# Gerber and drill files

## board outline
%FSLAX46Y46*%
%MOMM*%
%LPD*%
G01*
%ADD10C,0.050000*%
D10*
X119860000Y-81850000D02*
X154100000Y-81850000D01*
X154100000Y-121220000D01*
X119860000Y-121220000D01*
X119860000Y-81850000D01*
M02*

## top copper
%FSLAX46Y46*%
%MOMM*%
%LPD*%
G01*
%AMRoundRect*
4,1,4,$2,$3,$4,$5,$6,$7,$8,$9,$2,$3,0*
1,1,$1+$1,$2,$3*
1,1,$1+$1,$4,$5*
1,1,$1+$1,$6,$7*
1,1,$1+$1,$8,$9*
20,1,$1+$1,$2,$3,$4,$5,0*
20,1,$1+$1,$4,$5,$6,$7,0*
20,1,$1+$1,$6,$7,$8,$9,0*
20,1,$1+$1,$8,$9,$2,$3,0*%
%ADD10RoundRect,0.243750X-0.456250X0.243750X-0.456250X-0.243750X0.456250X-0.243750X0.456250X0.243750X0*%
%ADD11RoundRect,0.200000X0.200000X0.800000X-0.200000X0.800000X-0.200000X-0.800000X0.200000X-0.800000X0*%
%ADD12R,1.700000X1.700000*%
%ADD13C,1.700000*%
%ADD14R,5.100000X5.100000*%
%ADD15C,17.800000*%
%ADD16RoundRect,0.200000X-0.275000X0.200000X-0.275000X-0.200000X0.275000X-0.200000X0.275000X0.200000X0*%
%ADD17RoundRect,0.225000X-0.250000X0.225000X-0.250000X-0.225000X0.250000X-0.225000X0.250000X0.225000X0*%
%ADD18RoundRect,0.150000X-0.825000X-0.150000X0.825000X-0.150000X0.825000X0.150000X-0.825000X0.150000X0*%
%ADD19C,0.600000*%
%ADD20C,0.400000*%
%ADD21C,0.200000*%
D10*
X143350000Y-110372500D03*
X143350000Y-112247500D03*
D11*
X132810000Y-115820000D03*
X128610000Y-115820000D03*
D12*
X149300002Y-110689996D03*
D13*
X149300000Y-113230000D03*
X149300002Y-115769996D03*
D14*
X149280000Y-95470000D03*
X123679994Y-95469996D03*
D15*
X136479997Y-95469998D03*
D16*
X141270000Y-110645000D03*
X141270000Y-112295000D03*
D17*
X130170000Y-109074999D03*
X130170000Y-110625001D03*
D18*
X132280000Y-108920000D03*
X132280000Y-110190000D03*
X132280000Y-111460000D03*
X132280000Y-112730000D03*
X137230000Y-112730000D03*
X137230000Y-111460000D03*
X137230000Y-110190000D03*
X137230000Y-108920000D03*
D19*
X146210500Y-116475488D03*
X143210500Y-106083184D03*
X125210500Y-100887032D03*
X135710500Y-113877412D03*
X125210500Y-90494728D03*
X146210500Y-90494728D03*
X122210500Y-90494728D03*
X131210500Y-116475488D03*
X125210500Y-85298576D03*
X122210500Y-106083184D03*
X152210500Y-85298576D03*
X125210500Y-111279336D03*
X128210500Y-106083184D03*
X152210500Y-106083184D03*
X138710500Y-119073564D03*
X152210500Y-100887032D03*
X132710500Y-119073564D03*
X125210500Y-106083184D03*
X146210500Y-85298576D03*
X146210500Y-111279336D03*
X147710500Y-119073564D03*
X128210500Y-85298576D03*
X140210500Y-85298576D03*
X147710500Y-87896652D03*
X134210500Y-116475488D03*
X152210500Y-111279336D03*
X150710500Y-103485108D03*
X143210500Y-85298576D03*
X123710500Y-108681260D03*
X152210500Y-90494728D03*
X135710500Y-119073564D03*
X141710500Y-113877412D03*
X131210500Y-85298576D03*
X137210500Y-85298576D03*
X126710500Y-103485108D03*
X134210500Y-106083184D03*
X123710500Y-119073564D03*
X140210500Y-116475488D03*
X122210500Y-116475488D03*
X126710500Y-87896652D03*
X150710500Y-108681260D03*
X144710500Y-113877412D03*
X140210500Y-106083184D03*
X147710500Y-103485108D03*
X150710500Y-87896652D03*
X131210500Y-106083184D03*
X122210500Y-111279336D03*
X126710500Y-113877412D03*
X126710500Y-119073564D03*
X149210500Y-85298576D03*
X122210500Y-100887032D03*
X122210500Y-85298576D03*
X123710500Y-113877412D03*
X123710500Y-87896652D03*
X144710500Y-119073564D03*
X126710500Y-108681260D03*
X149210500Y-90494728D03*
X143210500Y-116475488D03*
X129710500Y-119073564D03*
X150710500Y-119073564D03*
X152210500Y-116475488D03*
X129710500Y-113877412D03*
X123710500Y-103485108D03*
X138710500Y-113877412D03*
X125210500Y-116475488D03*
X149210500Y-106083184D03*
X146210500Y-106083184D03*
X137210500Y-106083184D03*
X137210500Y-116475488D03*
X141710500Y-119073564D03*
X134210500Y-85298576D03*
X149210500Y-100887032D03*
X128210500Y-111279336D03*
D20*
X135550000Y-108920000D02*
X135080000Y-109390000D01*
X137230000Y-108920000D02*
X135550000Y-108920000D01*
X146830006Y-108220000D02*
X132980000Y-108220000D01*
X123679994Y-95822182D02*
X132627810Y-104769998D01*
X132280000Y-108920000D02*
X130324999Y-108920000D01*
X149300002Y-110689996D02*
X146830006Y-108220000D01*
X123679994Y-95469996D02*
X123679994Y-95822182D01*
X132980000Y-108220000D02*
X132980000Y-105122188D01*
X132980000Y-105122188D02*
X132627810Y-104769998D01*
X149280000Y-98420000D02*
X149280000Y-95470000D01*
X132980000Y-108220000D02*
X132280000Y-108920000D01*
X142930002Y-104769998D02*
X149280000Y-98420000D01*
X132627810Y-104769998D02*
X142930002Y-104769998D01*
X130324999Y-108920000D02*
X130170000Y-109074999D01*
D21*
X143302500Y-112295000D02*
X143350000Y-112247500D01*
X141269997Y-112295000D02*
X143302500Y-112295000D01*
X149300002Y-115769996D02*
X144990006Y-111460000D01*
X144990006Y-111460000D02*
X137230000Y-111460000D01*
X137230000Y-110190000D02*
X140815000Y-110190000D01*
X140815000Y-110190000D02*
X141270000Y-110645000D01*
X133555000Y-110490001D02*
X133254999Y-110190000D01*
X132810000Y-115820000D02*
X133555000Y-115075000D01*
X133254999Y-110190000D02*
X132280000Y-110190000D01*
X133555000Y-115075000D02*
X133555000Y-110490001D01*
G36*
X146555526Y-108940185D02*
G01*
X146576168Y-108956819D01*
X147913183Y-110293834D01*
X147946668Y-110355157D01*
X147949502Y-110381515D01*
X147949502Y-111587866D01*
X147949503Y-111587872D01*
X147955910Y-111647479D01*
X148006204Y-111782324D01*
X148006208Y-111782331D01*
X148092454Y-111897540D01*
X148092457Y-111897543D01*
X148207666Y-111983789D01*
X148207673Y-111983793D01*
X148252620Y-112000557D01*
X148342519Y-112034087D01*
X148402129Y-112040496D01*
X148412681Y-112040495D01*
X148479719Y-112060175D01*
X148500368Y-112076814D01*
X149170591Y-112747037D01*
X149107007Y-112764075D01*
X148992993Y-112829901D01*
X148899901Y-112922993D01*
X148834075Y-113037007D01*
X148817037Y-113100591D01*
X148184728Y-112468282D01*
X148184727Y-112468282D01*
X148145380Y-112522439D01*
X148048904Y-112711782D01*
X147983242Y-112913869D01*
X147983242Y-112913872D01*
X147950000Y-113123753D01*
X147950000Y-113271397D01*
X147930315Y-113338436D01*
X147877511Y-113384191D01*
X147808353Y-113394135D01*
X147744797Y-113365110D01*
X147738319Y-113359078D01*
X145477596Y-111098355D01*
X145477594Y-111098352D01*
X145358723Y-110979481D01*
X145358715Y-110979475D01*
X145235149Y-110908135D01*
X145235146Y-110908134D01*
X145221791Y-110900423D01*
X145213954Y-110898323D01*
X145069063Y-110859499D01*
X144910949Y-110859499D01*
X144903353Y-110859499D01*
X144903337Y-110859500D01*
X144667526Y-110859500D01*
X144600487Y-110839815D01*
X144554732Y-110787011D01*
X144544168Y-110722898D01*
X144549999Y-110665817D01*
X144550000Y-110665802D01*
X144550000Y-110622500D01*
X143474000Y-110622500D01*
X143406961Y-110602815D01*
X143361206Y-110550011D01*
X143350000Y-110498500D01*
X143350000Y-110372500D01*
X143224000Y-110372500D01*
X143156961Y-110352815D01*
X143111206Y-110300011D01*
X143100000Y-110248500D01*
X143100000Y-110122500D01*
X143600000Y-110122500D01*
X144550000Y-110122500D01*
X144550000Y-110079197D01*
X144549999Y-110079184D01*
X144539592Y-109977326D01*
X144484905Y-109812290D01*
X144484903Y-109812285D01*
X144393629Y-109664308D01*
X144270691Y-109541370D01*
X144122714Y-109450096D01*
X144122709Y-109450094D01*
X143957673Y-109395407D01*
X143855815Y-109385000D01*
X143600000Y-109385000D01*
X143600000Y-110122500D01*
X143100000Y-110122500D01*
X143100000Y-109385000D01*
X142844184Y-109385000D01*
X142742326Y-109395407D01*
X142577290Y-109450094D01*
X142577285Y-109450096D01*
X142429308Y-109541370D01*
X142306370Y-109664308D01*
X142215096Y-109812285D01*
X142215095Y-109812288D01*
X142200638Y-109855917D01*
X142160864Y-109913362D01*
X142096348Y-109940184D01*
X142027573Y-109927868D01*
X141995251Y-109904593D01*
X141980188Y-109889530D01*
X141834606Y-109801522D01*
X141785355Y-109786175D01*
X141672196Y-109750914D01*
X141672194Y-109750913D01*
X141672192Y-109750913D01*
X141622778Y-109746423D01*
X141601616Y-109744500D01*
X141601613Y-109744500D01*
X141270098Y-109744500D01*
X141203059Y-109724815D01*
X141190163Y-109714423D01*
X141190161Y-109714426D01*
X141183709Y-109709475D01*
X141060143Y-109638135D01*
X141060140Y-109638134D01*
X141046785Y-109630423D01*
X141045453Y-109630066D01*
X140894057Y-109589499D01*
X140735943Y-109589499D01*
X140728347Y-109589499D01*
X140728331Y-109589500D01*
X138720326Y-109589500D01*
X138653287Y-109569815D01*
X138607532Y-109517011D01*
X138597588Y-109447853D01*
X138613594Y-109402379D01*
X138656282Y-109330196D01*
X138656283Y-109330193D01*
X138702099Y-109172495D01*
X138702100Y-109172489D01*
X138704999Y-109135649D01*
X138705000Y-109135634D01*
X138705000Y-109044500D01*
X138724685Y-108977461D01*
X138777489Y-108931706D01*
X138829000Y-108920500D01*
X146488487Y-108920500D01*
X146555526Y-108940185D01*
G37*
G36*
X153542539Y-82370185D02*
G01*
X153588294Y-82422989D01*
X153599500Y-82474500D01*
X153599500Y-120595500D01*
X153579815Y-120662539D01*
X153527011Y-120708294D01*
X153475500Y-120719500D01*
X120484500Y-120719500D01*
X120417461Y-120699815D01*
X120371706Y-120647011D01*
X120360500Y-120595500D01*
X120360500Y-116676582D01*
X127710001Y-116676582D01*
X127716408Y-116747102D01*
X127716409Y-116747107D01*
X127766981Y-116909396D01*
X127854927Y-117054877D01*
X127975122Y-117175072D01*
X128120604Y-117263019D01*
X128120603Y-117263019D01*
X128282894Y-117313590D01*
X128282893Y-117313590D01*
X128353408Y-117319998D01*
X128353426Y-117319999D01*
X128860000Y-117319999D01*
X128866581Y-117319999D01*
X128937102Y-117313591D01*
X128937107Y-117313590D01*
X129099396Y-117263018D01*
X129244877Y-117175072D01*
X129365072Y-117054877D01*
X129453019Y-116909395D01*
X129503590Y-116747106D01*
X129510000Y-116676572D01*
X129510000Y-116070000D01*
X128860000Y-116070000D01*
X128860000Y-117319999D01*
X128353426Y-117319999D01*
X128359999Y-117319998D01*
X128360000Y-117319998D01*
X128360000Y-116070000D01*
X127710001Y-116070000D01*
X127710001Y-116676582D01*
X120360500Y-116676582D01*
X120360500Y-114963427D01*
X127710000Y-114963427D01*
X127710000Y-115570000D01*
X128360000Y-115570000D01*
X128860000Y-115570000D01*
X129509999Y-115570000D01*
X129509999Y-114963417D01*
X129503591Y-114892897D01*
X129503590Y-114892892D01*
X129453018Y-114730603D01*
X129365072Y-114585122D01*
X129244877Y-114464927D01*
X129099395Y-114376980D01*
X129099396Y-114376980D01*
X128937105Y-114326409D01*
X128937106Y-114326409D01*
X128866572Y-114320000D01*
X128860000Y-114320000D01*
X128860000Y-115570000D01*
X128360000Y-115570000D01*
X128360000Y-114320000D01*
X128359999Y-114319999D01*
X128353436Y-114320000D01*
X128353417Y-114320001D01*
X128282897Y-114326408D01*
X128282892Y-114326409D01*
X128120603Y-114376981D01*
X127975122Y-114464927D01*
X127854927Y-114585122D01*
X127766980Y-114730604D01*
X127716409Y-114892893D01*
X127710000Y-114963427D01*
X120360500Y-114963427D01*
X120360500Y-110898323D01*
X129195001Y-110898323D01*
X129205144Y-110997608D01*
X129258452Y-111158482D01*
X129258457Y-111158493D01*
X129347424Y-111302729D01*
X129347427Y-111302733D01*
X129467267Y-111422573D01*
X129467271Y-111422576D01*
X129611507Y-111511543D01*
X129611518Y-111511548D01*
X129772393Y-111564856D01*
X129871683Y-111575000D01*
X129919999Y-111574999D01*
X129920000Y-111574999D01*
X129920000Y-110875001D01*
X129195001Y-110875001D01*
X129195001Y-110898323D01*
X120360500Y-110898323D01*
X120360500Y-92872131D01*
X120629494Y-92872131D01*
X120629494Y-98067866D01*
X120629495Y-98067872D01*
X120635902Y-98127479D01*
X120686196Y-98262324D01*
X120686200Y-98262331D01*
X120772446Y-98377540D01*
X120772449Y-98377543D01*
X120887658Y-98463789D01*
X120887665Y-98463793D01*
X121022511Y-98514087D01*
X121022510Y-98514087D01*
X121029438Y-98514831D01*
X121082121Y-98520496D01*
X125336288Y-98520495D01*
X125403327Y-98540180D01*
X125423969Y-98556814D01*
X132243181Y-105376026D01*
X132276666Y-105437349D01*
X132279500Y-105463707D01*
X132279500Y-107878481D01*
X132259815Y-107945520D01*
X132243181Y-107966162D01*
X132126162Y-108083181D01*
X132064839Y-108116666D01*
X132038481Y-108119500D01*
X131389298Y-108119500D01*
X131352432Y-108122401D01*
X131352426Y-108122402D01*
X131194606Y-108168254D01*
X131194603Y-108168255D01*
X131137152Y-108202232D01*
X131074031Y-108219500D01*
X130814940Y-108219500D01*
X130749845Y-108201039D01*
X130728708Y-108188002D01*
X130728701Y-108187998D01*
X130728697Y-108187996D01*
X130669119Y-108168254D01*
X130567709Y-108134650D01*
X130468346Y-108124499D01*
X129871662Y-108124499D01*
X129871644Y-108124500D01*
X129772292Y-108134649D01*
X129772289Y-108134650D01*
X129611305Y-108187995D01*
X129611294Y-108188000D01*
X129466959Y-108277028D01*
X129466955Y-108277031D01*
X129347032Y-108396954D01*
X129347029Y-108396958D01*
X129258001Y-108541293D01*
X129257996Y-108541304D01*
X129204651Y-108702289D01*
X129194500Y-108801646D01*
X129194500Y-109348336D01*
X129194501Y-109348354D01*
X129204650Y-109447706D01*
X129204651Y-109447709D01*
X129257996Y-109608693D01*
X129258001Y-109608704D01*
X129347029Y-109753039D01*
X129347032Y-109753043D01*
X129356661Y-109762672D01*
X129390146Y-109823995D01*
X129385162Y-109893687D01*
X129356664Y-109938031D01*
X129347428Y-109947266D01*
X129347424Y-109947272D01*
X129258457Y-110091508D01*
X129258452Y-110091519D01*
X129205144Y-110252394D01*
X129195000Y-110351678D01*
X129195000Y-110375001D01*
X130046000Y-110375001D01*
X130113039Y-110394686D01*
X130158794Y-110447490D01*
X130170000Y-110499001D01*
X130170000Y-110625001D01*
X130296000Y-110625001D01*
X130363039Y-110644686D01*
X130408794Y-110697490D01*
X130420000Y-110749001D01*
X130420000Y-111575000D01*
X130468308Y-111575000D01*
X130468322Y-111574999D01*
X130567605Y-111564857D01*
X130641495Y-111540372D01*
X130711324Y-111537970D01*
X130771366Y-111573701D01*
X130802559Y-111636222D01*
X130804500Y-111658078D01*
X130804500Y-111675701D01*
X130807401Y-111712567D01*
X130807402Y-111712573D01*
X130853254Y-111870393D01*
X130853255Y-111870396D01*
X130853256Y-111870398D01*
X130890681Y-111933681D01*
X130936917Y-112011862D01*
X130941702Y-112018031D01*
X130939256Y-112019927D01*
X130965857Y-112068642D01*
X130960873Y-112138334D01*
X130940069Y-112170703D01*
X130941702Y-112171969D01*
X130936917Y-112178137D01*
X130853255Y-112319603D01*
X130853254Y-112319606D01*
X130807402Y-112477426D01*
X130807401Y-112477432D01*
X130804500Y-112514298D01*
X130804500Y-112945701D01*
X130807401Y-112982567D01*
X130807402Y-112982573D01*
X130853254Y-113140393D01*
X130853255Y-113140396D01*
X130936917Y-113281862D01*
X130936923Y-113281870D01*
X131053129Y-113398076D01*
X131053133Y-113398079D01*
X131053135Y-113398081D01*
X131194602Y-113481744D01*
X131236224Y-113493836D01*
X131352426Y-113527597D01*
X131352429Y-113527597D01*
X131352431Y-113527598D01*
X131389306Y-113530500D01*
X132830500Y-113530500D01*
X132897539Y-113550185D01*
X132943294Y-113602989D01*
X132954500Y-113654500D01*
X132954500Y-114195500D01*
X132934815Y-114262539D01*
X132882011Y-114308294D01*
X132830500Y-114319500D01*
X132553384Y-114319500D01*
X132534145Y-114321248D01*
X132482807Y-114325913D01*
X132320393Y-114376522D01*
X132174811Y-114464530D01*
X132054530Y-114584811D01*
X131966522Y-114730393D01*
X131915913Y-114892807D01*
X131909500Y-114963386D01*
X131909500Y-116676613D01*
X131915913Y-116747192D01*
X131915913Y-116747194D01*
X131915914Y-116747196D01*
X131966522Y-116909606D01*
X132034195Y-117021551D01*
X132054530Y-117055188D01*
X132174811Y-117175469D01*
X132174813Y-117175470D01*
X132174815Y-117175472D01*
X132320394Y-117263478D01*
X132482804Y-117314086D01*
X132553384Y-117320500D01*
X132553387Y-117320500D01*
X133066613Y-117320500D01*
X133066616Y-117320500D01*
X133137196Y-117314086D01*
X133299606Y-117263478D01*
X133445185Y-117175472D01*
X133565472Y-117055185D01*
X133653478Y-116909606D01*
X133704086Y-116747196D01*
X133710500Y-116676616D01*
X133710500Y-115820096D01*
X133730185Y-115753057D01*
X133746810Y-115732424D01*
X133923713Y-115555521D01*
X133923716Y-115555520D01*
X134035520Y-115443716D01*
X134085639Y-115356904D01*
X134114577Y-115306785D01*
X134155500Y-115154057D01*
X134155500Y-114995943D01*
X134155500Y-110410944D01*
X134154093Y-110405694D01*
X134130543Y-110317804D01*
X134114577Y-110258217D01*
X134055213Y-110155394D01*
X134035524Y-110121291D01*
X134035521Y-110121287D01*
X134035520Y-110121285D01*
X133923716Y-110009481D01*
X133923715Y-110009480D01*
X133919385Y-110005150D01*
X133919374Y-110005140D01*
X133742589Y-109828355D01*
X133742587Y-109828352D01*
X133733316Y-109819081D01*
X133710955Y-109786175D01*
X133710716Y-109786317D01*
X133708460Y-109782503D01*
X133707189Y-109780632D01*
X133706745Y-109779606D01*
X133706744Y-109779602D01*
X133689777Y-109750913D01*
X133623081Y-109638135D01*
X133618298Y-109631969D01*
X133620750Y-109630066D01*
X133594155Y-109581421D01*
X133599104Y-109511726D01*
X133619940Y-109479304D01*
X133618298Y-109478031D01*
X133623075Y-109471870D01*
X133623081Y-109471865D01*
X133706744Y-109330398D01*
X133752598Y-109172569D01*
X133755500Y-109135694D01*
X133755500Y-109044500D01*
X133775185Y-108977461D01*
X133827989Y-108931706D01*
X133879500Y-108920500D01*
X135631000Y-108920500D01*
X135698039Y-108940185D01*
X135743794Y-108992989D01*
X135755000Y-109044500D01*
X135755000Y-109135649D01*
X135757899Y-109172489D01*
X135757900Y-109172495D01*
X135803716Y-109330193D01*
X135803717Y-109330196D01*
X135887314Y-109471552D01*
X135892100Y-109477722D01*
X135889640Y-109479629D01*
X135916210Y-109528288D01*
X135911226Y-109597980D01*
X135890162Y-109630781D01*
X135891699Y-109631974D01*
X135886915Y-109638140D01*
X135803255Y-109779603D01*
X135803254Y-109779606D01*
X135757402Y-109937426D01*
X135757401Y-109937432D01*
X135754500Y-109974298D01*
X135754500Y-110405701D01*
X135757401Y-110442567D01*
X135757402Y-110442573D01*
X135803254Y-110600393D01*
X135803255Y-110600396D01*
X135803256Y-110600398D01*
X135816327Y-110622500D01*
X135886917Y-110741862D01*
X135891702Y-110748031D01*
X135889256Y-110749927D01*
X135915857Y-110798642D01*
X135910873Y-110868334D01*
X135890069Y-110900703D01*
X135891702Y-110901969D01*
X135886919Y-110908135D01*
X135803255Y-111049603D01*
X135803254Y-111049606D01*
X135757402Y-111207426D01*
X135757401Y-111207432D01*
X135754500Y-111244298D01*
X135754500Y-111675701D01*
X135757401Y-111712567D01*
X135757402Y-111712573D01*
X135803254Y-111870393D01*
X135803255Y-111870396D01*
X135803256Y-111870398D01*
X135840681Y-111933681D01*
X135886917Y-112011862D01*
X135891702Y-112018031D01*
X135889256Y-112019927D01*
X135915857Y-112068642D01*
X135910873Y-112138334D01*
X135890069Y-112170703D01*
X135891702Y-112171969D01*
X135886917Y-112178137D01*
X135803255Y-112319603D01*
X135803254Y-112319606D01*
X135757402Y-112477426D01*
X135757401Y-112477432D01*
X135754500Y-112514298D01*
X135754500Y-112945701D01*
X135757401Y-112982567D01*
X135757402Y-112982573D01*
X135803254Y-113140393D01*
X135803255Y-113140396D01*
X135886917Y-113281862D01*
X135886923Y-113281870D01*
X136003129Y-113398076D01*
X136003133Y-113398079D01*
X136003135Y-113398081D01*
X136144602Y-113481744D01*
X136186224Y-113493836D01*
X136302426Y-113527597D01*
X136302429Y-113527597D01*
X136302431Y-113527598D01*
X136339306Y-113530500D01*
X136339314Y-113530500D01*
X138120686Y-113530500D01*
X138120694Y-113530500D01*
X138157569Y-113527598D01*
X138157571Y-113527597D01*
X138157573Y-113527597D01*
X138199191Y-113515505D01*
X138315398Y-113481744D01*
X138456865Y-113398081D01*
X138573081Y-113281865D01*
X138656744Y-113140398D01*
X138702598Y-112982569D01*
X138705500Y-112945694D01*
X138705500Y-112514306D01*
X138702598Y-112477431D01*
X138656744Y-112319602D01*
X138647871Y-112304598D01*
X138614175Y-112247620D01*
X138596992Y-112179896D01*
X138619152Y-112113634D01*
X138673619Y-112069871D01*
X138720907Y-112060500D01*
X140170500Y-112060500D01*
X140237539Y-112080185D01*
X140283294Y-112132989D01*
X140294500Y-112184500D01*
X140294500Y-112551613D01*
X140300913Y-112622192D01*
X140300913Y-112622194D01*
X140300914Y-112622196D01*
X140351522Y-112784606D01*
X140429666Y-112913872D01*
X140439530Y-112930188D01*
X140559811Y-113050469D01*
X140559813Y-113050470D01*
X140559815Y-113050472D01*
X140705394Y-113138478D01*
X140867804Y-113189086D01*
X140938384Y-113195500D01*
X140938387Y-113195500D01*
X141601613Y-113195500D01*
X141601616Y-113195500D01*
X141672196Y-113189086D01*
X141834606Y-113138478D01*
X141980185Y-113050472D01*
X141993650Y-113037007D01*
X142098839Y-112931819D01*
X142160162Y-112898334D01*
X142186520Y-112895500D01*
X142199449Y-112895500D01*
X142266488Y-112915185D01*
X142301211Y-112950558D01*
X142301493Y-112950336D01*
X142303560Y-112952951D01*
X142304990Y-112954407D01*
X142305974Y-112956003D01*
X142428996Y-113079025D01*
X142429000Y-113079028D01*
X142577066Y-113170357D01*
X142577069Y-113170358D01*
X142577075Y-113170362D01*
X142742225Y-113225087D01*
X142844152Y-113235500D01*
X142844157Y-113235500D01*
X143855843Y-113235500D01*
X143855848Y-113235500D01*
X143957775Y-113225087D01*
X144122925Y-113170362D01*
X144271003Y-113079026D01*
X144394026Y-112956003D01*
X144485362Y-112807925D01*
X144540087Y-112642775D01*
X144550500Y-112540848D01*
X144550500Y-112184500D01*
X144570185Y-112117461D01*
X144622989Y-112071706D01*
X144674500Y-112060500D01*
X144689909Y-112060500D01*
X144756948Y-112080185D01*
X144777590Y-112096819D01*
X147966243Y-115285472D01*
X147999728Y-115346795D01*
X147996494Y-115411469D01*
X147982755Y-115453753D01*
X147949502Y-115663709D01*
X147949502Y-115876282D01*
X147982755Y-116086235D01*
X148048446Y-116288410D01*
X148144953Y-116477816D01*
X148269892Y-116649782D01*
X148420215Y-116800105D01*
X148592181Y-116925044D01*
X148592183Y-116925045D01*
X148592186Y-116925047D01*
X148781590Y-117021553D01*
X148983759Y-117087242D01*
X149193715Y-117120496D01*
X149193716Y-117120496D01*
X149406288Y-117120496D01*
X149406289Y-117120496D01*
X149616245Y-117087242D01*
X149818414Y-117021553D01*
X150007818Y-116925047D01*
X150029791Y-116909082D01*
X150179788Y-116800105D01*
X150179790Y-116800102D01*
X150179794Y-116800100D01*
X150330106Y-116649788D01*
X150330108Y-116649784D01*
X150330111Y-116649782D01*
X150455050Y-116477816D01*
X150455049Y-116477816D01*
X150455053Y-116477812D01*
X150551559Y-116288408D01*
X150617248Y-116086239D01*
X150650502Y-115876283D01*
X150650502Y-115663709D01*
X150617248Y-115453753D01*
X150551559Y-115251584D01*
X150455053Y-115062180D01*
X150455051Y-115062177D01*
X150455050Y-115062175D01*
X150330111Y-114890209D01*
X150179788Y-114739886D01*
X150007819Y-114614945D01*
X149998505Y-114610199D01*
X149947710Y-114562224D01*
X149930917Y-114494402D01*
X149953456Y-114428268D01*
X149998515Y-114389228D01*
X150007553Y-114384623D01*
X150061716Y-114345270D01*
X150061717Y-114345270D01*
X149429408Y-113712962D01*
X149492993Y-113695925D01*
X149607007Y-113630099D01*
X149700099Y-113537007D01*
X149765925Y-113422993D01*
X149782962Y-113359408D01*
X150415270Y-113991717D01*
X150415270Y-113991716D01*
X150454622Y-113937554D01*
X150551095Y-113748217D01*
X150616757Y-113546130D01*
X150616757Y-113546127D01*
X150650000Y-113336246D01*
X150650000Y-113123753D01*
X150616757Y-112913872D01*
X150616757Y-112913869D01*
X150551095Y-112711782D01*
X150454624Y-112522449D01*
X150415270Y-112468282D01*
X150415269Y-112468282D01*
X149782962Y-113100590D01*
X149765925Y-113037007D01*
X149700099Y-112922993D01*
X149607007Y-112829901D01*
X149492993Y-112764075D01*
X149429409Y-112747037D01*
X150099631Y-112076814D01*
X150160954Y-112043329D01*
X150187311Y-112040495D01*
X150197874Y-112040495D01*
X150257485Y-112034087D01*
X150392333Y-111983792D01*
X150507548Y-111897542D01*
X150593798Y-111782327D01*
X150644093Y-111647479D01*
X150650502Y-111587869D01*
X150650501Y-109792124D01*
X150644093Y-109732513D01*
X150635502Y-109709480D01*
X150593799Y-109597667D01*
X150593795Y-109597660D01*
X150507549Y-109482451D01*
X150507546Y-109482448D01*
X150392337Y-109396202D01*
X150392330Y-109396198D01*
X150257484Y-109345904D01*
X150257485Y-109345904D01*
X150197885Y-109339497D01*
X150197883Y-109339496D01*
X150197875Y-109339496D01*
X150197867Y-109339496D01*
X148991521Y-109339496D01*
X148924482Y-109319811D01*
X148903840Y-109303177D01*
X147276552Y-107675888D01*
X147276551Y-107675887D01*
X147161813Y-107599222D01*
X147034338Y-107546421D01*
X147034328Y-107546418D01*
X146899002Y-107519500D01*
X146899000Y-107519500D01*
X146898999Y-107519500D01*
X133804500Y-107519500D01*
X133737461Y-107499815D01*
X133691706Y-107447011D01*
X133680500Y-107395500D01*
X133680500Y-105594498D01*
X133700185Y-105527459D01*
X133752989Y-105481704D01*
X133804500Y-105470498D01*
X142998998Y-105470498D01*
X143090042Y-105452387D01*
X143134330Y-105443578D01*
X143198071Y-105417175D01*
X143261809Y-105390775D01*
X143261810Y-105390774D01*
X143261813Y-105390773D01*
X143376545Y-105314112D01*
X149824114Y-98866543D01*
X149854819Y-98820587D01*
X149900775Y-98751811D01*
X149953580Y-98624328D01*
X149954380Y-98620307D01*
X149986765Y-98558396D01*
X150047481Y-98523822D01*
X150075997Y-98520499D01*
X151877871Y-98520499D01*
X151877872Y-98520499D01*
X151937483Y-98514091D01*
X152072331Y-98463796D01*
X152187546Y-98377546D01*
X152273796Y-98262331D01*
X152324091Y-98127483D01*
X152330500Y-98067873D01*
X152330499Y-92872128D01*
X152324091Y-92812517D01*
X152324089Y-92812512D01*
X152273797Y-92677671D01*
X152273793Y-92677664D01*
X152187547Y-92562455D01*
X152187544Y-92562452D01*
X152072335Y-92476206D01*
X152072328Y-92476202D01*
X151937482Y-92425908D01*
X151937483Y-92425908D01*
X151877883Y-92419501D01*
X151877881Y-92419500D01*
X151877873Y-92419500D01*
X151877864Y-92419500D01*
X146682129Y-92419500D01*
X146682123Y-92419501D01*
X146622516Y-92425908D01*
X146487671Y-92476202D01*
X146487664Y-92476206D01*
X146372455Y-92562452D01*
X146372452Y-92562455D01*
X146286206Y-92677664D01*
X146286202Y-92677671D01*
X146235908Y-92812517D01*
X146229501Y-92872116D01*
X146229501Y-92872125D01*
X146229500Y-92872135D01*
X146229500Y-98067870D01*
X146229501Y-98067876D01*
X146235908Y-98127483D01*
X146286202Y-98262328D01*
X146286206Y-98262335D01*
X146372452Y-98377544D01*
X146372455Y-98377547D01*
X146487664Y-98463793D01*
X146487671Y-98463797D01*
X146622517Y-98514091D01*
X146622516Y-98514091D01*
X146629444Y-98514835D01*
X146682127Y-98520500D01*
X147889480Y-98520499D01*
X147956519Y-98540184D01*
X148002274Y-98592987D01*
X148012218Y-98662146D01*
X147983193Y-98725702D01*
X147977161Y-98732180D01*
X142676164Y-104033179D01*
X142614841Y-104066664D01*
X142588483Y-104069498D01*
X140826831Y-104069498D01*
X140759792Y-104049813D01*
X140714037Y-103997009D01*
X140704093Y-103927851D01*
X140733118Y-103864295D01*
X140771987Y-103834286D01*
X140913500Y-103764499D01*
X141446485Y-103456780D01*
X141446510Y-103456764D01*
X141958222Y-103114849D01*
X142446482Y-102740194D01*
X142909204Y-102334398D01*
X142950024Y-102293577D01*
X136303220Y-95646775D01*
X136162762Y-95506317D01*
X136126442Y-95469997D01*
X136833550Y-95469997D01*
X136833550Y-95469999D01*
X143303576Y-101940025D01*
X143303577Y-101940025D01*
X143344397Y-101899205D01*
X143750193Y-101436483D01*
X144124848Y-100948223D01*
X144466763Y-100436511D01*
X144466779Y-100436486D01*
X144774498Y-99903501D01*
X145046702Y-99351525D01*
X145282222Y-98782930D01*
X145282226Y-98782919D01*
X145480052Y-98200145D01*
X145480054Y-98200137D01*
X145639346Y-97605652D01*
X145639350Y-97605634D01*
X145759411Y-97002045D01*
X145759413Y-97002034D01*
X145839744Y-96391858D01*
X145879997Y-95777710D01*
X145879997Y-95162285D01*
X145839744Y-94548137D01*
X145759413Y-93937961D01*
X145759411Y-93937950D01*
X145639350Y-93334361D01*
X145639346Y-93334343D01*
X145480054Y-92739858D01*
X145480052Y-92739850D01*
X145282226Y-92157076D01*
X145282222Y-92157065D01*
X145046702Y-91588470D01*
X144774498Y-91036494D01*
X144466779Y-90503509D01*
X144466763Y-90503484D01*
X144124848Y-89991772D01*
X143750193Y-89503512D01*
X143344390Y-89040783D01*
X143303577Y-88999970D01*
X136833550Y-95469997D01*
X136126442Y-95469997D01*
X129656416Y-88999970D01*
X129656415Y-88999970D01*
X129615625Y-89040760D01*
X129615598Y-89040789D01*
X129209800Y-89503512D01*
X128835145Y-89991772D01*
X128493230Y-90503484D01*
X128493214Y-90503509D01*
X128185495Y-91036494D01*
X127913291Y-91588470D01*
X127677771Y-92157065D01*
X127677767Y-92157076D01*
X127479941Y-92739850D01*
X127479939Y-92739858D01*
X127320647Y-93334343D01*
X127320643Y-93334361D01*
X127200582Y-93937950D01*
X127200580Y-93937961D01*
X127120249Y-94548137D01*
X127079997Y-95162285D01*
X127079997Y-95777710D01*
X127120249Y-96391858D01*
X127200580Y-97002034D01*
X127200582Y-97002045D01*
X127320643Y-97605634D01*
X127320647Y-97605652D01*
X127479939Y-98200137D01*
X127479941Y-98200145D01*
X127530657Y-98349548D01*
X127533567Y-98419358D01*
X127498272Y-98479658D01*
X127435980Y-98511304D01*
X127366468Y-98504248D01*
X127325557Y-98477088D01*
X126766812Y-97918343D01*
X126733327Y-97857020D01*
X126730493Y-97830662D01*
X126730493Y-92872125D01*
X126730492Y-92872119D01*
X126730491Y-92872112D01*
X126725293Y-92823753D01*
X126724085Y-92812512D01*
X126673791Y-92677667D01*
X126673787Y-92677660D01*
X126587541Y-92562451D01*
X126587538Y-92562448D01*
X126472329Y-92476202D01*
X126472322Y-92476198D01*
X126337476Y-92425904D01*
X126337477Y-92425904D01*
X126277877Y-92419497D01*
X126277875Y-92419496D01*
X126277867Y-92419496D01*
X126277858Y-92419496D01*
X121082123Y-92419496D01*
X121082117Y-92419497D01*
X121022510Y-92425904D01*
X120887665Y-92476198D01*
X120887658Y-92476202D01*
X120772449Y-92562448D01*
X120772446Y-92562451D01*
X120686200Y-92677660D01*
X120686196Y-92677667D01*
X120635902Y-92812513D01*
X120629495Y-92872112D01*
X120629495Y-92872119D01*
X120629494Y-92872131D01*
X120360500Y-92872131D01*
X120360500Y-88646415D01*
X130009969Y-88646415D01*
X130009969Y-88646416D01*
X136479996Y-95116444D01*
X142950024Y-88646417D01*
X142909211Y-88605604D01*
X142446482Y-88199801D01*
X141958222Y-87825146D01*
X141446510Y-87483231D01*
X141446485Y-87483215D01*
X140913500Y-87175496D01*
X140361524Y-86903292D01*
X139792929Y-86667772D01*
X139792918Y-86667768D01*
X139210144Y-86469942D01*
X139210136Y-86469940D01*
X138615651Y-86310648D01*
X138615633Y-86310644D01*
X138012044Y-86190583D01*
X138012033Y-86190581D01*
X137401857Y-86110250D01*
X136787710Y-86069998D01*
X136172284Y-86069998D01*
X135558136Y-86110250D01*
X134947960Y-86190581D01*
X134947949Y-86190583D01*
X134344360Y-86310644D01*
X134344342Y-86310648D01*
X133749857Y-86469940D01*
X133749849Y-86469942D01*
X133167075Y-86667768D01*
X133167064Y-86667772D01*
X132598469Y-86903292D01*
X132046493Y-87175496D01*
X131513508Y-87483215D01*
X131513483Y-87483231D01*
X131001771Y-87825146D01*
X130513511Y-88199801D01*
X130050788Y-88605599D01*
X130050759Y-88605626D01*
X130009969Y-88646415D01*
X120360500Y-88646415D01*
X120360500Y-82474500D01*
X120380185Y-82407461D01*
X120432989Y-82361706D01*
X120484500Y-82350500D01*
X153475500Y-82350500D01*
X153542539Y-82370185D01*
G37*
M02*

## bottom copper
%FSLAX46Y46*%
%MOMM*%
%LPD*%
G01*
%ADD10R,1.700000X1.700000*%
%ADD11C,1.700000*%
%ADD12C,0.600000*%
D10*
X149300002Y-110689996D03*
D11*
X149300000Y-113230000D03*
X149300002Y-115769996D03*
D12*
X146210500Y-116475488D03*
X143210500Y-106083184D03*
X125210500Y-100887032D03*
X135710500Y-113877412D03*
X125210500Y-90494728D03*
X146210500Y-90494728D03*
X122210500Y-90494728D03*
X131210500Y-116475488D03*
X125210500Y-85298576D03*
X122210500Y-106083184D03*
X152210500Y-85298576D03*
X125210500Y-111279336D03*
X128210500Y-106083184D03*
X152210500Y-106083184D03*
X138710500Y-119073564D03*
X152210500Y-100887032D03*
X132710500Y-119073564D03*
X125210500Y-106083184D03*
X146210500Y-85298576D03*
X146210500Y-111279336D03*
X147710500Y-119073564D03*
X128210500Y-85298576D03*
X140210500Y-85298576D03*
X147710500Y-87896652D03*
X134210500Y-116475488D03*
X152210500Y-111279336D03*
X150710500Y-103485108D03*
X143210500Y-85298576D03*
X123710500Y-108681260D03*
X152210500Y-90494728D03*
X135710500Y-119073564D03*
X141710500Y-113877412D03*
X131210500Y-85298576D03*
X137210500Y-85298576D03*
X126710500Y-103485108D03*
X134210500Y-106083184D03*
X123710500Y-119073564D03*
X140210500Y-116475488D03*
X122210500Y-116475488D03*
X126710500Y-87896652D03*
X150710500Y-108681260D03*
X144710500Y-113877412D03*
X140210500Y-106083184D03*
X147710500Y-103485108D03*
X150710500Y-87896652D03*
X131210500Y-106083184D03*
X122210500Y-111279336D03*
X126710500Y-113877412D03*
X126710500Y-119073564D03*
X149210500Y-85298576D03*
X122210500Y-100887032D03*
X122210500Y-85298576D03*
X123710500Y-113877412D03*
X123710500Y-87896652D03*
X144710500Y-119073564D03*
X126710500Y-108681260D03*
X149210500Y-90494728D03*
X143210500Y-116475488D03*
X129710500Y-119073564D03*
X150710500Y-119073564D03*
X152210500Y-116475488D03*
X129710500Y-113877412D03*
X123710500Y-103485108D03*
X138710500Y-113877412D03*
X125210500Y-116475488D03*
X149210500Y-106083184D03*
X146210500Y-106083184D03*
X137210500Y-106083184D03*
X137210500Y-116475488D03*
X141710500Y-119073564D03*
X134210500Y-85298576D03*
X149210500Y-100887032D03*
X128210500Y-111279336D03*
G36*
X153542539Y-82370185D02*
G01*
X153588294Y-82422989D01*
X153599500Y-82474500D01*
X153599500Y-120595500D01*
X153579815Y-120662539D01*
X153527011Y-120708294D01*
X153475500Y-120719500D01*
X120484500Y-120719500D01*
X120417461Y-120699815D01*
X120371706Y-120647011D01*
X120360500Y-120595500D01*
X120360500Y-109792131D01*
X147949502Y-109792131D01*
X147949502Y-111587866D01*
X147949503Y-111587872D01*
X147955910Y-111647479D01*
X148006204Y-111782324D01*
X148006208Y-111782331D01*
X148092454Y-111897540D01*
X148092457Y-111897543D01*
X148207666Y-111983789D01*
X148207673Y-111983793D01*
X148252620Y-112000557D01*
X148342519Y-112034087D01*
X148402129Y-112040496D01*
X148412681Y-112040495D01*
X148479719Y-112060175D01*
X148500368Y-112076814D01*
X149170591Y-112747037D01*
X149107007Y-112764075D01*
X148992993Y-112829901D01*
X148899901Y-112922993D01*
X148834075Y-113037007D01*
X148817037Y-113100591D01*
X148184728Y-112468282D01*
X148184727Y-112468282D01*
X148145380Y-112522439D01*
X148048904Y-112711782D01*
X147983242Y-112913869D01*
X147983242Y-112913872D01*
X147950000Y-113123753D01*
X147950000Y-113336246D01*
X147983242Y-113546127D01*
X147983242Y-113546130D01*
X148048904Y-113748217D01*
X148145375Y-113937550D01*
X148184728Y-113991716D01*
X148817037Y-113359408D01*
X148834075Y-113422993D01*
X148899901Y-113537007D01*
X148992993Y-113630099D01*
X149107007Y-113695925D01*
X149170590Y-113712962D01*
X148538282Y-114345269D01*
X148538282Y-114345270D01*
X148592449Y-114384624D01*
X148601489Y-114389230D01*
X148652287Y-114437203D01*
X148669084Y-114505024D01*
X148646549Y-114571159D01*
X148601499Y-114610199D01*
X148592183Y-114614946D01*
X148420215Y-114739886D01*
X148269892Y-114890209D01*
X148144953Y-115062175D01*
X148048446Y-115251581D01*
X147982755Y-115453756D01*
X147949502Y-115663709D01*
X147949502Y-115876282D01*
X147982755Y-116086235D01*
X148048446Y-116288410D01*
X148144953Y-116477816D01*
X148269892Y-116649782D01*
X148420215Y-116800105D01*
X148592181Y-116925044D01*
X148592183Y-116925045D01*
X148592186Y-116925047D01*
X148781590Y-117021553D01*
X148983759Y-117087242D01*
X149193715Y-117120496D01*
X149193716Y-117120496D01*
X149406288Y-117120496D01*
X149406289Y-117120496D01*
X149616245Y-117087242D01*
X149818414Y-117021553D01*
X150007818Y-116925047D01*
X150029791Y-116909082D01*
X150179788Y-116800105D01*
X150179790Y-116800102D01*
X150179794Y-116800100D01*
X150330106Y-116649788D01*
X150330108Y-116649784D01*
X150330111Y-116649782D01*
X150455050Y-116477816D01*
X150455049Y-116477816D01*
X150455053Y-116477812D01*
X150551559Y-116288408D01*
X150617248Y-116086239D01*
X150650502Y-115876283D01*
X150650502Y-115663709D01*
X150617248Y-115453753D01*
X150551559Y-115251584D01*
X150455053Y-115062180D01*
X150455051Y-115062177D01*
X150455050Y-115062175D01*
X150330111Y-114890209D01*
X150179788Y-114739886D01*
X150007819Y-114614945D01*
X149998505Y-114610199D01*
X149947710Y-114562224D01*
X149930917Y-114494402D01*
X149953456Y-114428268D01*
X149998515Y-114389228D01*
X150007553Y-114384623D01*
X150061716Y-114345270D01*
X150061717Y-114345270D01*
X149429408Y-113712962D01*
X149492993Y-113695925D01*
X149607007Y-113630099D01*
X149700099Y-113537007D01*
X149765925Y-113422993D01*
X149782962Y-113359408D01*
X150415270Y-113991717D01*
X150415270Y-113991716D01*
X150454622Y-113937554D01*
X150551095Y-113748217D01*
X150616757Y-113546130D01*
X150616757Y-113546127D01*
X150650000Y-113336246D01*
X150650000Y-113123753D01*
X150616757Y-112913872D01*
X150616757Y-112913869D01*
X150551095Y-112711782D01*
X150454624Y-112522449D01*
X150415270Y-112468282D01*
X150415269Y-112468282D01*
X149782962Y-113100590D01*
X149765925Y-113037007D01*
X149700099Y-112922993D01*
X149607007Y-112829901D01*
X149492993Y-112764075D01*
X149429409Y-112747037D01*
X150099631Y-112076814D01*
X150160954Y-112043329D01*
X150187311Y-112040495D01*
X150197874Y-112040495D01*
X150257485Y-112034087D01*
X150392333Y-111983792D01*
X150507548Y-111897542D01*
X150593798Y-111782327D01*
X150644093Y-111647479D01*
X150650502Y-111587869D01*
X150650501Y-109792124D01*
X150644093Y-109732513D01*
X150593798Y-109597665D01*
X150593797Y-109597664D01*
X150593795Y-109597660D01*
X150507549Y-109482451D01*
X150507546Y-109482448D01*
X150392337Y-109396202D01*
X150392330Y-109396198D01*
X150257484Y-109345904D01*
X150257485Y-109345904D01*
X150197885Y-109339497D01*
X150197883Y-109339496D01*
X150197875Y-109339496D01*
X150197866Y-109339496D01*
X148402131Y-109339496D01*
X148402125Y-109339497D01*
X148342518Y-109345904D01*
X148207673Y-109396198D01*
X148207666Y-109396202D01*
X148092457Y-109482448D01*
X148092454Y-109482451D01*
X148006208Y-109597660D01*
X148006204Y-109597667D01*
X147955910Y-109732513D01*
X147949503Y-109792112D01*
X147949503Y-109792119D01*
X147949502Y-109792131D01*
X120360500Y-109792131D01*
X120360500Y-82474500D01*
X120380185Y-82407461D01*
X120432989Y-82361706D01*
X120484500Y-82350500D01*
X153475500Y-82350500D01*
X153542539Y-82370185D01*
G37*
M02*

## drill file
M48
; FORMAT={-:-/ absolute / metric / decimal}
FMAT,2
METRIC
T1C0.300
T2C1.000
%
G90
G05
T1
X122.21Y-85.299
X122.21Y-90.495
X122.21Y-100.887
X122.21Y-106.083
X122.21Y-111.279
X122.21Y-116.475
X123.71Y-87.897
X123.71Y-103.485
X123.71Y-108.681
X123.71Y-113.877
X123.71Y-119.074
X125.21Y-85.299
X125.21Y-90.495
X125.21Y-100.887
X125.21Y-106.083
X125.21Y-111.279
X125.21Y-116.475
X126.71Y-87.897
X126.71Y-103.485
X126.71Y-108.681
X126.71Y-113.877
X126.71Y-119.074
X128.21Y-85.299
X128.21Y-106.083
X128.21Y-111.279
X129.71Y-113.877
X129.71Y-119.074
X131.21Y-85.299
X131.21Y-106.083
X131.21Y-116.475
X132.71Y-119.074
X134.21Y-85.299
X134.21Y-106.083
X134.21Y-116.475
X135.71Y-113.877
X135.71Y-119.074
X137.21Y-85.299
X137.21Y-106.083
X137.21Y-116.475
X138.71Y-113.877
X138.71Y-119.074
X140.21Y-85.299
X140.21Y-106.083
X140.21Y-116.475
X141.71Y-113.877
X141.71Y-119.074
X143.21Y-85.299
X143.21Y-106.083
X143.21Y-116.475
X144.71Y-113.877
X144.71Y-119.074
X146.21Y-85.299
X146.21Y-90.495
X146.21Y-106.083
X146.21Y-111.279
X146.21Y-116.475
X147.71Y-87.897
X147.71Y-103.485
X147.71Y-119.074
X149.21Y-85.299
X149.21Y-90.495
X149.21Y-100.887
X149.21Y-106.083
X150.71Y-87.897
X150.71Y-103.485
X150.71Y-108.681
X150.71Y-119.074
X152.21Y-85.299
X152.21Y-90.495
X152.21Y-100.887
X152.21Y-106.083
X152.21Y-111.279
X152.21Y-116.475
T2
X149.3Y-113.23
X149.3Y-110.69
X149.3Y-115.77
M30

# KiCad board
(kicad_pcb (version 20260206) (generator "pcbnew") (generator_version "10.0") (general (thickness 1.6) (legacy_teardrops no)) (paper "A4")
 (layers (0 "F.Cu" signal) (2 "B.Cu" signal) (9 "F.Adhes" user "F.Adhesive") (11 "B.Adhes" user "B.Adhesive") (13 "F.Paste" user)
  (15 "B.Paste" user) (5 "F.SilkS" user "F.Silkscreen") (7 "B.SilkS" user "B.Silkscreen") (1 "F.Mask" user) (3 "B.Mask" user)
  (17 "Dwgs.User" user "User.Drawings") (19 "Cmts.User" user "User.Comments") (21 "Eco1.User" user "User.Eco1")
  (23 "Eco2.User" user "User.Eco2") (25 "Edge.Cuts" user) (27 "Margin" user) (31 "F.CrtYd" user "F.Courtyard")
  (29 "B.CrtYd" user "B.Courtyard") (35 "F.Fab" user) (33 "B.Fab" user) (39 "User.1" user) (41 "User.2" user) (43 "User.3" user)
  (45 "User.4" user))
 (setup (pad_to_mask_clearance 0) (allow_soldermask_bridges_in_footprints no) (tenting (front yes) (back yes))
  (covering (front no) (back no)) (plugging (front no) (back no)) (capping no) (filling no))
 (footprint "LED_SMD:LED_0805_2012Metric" (layer "F.Cu") (at 143.35 111.31 -90)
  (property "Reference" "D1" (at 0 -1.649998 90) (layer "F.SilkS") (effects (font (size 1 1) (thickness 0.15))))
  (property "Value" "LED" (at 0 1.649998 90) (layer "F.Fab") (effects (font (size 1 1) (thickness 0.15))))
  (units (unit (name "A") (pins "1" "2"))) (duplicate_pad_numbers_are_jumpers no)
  (pad "1" smd roundrect (at -0.9375 0 270) (size 0.975 1.4) (layers "F.Cu" "F.Mask" "F.Paste") (roundrect_rratio 0.25) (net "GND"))
  (pad "2" smd roundrect (at 0.9375 0 270) (size 0.975 1.4) (layers "F.Cu" "F.Mask" "F.Paste") (roundrect_rratio 0.25) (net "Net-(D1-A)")))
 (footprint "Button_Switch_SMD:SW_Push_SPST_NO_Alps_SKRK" (layer "F.Cu") (at 130.71 115.82 180)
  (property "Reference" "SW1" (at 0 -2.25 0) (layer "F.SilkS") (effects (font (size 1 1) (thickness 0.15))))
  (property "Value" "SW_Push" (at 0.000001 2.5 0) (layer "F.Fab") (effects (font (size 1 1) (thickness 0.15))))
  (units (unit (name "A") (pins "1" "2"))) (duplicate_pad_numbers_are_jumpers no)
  (pad "1" smd roundrect (at -2.1 0 180) (size 0.8 2) (layers "F.Cu" "F.Mask" "F.Paste") (roundrect_rratio 0.25) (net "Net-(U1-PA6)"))
  (pad "2" smd roundrect (at 2.1 0 180) (size 0.8 2) (layers "F.Cu" "F.Mask" "F.Paste") (roundrect_rratio 0.25) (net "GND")))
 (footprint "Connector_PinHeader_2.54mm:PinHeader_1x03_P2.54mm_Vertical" (layer "F.Cu") (at 149.300002 110.689996)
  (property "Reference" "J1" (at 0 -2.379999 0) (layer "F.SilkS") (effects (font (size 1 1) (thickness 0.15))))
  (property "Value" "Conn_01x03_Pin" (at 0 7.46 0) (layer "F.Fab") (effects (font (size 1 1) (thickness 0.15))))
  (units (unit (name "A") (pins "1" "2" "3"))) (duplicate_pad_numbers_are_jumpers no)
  (pad "1" thru_hole rect (at 0 0) (size 1.7 1.7) (drill 1) (layers "*.Cu" "*.Mask") (remove_unused_layers no) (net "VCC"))
  (pad "2" thru_hole circle (at -0.000002 2.540004) (size 1.7 1.7) (drill 1) (layers "*.Cu" "*.Mask") (remove_unused_layers no) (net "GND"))
  (pad "3" thru_hole circle (at 0 5.08) (size 1.7 1.7) (drill 1) (layers "*.Cu" "*.Mask") (remove_unused_layers no) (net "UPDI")))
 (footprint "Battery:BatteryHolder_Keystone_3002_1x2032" (layer "F.Cu") (at 136.479997 95.469998 180)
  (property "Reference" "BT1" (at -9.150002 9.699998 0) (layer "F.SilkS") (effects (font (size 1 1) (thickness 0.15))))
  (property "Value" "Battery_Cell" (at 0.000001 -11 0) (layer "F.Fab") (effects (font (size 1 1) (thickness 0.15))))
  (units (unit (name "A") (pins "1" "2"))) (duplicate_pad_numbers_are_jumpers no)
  (pad "1" smd rect (at -12.800003 -0.000002 180) (size 5.1 5.1) (layers "F.Cu" "F.Mask" "F.Paste") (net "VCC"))
  (pad "1" smd rect (at 12.800003 0.000002 180) (size 5.1 5.1) (layers "F.Cu" "F.Mask" "F.Paste") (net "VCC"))
  (pad "2" smd circle (at 0 0 180) (size 17.8 17.8) (layers "F.Cu" "F.Mask") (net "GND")))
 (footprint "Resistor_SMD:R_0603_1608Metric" (layer "F.Cu") (at 141.27 111.47 -90)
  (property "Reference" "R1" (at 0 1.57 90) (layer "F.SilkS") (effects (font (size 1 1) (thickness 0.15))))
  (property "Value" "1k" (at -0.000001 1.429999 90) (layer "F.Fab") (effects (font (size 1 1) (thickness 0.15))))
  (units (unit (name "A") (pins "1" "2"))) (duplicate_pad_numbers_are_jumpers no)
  (pad "1" smd roundrect (at -0.825 0 270) (size 0.8 0.95) (layers "F.Cu" "F.Mask" "F.Paste") (roundrect_rratio 0.25) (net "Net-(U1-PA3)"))
  (pad "2" smd roundrect (at 0.825 0 270) (size 0.8 0.95) (layers "F.Cu" "F.Mask" "F.Paste") (roundrect_rratio 0.25) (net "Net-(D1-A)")))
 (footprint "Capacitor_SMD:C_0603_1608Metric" (layer "F.Cu") (at 130.17 109.85 -90)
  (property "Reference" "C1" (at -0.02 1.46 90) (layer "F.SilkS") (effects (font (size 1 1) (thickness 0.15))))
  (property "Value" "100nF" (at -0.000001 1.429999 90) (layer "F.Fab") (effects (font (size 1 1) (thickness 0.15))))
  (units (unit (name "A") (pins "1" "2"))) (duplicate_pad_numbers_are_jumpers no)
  (pad "1" smd roundrect (at -0.775001 0 270) (size 0.9 0.95) (layers "F.Cu" "F.Mask" "F.Paste") (roundrect_rratio 0.25) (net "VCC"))
  (pad "2" smd roundrect (at 0.775001 0 270) (size 0.9 0.95) (layers "F.Cu" "F.Mask" "F.Paste") (roundrect_rratio 0.25) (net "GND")))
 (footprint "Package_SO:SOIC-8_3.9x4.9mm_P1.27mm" (layer "F.Cu") (at 134.755 110.825)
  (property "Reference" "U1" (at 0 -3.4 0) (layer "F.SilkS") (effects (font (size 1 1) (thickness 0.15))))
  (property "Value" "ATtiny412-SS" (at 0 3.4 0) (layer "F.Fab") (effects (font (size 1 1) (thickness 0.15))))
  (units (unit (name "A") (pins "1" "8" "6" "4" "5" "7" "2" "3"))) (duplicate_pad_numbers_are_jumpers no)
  (pad "1" smd roundrect (at -2.475 -1.905) (size 1.95 0.6) (layers "F.Cu" "F.Mask" "F.Paste") (roundrect_rratio 0.25) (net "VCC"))
  (pad "2" smd roundrect (at -2.475 -0.635) (size 1.95 0.6) (layers "F.Cu" "F.Mask" "F.Paste") (roundrect_rratio 0.25) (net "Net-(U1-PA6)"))
  (pad "3" smd roundrect (at -2.475 0.635) (size 1.95 0.6) (layers "F.Cu" "F.Mask" "F.Paste") (roundrect_rratio 0.25)
   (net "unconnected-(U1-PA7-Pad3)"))
  (pad "4" smd roundrect (at -2.475 1.905) (size 1.95 0.6) (layers "F.Cu" "F.Mask" "F.Paste") (roundrect_rratio 0.25)
   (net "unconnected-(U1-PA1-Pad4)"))
  (pad "5" smd roundrect (at 2.475 1.905) (size 1.95 0.6) (layers "F.Cu" "F.Mask" "F.Paste") (roundrect_rratio 0.25)
   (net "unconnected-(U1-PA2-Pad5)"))
  (pad "6" smd roundrect (at 2.475 0.635) (size 1.95 0.6) (layers "F.Cu" "F.Mask" "F.Paste") (roundrect_rratio 0.25) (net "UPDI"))
  (pad "7" smd roundrect (at 2.475 -0.635) (size 1.95 0.6) (layers "F.Cu" "F.Mask" "F.Paste") (roundrect_rratio 0.25) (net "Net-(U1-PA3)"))
  (pad "8" smd roundrect (at 2.475 -1.905) (size 1.95 0.6) (layers "F.Cu" "F.Mask" "F.Paste") (roundrect_rratio 0.25) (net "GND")))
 (gr_rect (start 119.86 81.85) (end 154.1 121.22) (stroke (width 0.05) (type default)) (fill no) (layer "Edge.Cuts"))
 (segment (start 135.55 108.92) (end 135.08 109.39) (width 0.4) (layer "F.Cu") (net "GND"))
 (segment (start 137.23 108.92) (end 135.55 108.92) (width 0.4) (layer "F.Cu") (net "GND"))
 (via (at 146.2105 116.475488) (size 0.6) (drill 0.3) (layers "F.Cu" "B.Cu") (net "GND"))
 (via (at 143.2105 106.083184) (size 0.6) (drill 0.3) (layers "F.Cu" "B.Cu") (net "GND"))
 (via (at 125.2105 100.887032) (size 0.6) (drill 0.3) (layers "F.Cu" "B.Cu") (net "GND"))
 (via (at 135.7105 113.877412) (size 0.6) (drill 0.3) (layers "F.Cu" "B.Cu") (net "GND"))
 (via (at 125.2105 90.494728) (size 0.6) (drill 0.3) (layers "F.Cu" "B.Cu") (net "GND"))
 (via (at 146.2105 90.494728) (size 0.6) (drill 0.3) (layers "F.Cu" "B.Cu") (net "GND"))
 (via (at 122.2105 90.494728) (size 0.6) (drill 0.3) (layers "F.Cu" "B.Cu") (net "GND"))
 (via (at 131.2105 116.475488) (size 0.6) (drill 0.3) (layers "F.Cu" "B.Cu") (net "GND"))
 (via (at 125.2105 85.298576) (size 0.6) (drill 0.3) (layers "F.Cu" "B.Cu") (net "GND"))
 (via (at 122.2105 106.083184) (size 0.6) (drill 0.3) (layers "F.Cu" "B.Cu") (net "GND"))
 (via (at 152.2105 85.298576) (size 0.6) (drill 0.3) (layers "F.Cu" "B.Cu") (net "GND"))
 (via (at 125.2105 111.279336) (size 0.6) (drill 0.3) (layers "F.Cu" "B.Cu") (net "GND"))
 (via (at 128.2105 106.083184) (size 0.6) (drill 0.3) (layers "F.Cu" "B.Cu") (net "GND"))
 (via (at 152.2105 106.083184) (size 0.6) (drill 0.3) (layers "F.Cu" "B.Cu") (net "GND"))
 (via (at 138.7105 119.073564) (size 0.6) (drill 0.3) (layers "F.Cu" "B.Cu") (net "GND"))
 (via (at 152.2105 100.887032) (size 0.6) (drill 0.3) (layers "F.Cu" "B.Cu") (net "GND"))
 (via (at 132.7105 119.073564) (size 0.6) (drill 0.3) (layers "F.Cu" "B.Cu") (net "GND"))
 (via (at 125.2105 106.083184) (size 0.6) (drill 0.3) (layers "F.Cu" "B.Cu") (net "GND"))
 (via (at 146.2105 85.298576) (size 0.6) (drill 0.3) (layers "F.Cu" "B.Cu") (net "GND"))
 (via (at 146.2105 111.279336) (size 0.6) (drill 0.3) (layers "F.Cu" "B.Cu") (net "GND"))
 (via (at 147.7105 119.073564) (size 0.6) (drill 0.3) (layers "F.Cu" "B.Cu") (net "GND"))
 (via (at 128.2105 85.298576) (size 0.6) (drill 0.3) (layers "F.Cu" "B.Cu") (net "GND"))
 (via (at 140.2105 85.298576) (size 0.6) (drill 0.3) (layers "F.Cu" "B.Cu") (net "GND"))
 (via (at 147.7105 87.896652) (size 0.6) (drill 0.3) (layers "F.Cu" "B.Cu") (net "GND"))
 (via (at 134.2105 116.475488) (size 0.6) (drill 0.3) (layers "F.Cu" "B.Cu") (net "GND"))
 (via (at 152.2105 111.279336) (size 0.6) (drill 0.3) (layers "F.Cu" "B.Cu") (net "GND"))
 (via (at 150.7105 103.485108) (size 0.6) (drill 0.3) (layers "F.Cu" "B.Cu") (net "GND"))
 (via (at 143.2105 85.298576) (size 0.6) (drill 0.3) (layers "F.Cu" "B.Cu") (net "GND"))
 (via (at 123.7105 108.68126) (size 0.6) (drill 0.3) (layers "F.Cu" "B.Cu") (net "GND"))
 (via (at 152.2105 90.494728) (size 0.6) (drill 0.3) (layers "F.Cu" "B.Cu") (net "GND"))
 (via (at 135.7105 119.073564) (size 0.6) (drill 0.3) (layers "F.Cu" "B.Cu") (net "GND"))
 (via (at 141.7105 113.877412) (size 0.6) (drill 0.3) (layers "F.Cu" "B.Cu") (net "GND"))
 (via (at 131.2105 85.298576) (size 0.6) (drill 0.3) (layers "F.Cu" "B.Cu") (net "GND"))
 (via (at 137.2105 85.298576) (size 0.6) (drill 0.3) (layers "F.Cu" "B.Cu") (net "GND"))
 (via (at 126.7105 103.485108) (size 0.6) (drill 0.3) (layers "F.Cu" "B.Cu") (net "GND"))
 (via (at 134.2105 106.083184) (size 0.6) (drill 0.3) (layers "F.Cu" "B.Cu") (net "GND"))
 (via (at 123.7105 119.073564) (size 0.6) (drill 0.3) (layers "F.Cu" "B.Cu") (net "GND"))
 (via (at 140.2105 116.475488) (size 0.6) (drill 0.3) (layers "F.Cu" "B.Cu") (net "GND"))
 (via (at 122.2105 116.475488) (size 0.6) (drill 0.3) (layers "F.Cu" "B.Cu") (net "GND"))
 (via (at 126.7105 87.896652) (size 0.6) (drill 0.3) (layers "F.Cu" "B.Cu") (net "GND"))
 (via (at 150.7105 108.68126) (size 0.6) (drill 0.3) (layers "F.Cu" "B.Cu") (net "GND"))
 (via (at 144.7105 113.877412) (size 0.6) (drill 0.3) (layers "F.Cu" "B.Cu") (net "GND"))
 (via (at 140.2105 106.083184) (size 0.6) (drill 0.3) (layers "F.Cu" "B.Cu") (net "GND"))
 (via (at 147.7105 103.485108) (size 0.6) (drill 0.3) (layers "F.Cu" "B.Cu") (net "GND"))
 (via (at 150.7105 87.896652) (size 0.6) (drill 0.3) (layers "F.Cu" "B.Cu") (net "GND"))
 (via (at 131.2105 106.083184) (size 0.6) (drill 0.3) (layers "F.Cu" "B.Cu") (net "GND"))
 (via (at 122.2105 111.279336) (size 0.6) (drill 0.3) (layers "F.Cu" "B.Cu") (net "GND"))
 (via (at 126.7105 113.877412) (size 0.6) (drill 0.3) (layers "F.Cu" "B.Cu") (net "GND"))
 (via (at 126.7105 119.073564) (size 0.6) (drill 0.3) (layers "F.Cu" "B.Cu") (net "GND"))
 (via (at 149.2105 85.298576) (size 0.6) (drill 0.3) (layers "F.Cu" "B.Cu") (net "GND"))
 (via (at 122.2105 100.887032) (size 0.6) (drill 0.3) (layers "F.Cu" "B.Cu") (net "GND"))
 (via (at 122.2105 85.298576) (size 0.6) (drill 0.3) (layers "F.Cu" "B.Cu") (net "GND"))
 (via (at 123.7105 113.877412) (size 0.6) (drill 0.3) (layers "F.Cu" "B.Cu") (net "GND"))
 (via (at 123.7105 87.896652) (size 0.6) (drill 0.3) (layers "F.Cu" "B.Cu") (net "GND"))
 (via (at 144.7105 119.073564) (size 0.6) (drill 0.3) (layers "F.Cu" "B.Cu") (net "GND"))
 (via (at 126.7105 108.68126) (size 0.6) (drill 0.3) (layers "F.Cu" "B.Cu") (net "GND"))
 (via (at 149.2105 90.494728) (size 0.6) (drill 0.3) (layers "F.Cu" "B.Cu") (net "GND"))
 (via (at 143.2105 116.475488) (size 0.6) (drill 0.3) (layers "F.Cu" "B.Cu") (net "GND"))
 (via (at 129.7105 119.073564) (size 0.6) (drill 0.3) (layers "F.Cu" "B.Cu") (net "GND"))
 (via (at 150.7105 119.073564) (size 0.6) (drill 0.3) (layers "F.Cu" "B.Cu") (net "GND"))
 (via (at 152.2105 116.475488) (size 0.6) (drill 0.3) (layers "F.Cu" "B.Cu") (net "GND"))
 (via (at 129.7105 113.877412) (size 0.6) (drill 0.3) (layers "F.Cu" "B.Cu") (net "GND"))
 (via (at 123.7105 103.485108) (size 0.6) (drill 0.3) (layers "F.Cu" "B.Cu") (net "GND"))
 (via (at 138.7105 113.877412) (size 0.6) (drill 0.3) (layers "F.Cu" "B.Cu") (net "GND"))
 (via (at 125.2105 116.475488) (size 0.6) (drill 0.3) (layers "F.Cu" "B.Cu") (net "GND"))
 (via (at 149.2105 106.083184) (size 0.6) (drill 0.3) (layers "F.Cu" "B.Cu") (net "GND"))
 (via (at 146.2105 106.083184) (size 0.6) (drill 0.3) (layers "F.Cu" "B.Cu") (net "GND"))
 (via (at 137.2105 106.083184) (size 0.6) (drill 0.3) (layers "F.Cu" "B.Cu") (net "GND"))
 (via (at 137.2105 116.475488) (size 0.6) (drill 0.3) (layers "F.Cu" "B.Cu") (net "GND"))
 (via (at 141.7105 119.073564) (size 0.6) (drill 0.3) (layers "F.Cu" "B.Cu") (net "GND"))
 (via (at 134.2105 85.298576) (size 0.6) (drill 0.3) (layers "F.Cu" "B.Cu") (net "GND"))
 (via (at 149.2105 100.887032) (size 0.6) (drill 0.3) (layers "F.Cu" "B.Cu") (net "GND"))
 (via (at 128.2105 111.279336) (size 0.6) (drill 0.3) (layers "F.Cu" "B.Cu") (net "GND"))
 (segment (start 146.830006 108.22) (end 132.98 108.22) (width 0.4) (layer "F.Cu") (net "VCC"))
 (segment (start 123.679994 95.822182) (end 132.62781 104.769998) (width 0.4) (layer "F.Cu") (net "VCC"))
 (segment (start 132.28 108.92) (end 130.324999 108.92) (width 0.4) (layer "F.Cu") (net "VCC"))
 (segment (start 149.300002 110.689996) (end 146.830006 108.22) (width 0.4) (layer "F.Cu") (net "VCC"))
 (segment (start 123.679994 95.469996) (end 123.679994 95.822182) (width 0.4) (layer "F.Cu") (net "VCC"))
 (segment (start 132.98 108.22) (end 132.98 105.122188) (width 0.4) (layer "F.Cu") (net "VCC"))
 (segment (start 132.98 105.122188) (end 132.62781 104.769998) (width 0.4) (layer "F.Cu") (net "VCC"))
 (segment (start 149.28 98.42) (end 149.28 95.47) (width 0.4) (layer "F.Cu") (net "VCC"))
 (segment (start 132.98 108.22) (end 132.28 108.92) (width 0.4) (layer "F.Cu") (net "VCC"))
 (segment (start 142.930002 104.769998) (end 149.28 98.42) (width 0.4) (layer "F.Cu") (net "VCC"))
 (segment (start 132.62781 104.769998) (end 142.930002 104.769998) (width 0.4) (layer "F.Cu") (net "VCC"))
 (segment (start 130.324999 108.92) (end 130.17 109.074999) (width 0.4) (layer "F.Cu") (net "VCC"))
 (segment (start 143.3025 112.295) (end 143.35 112.2475) (width 0.2) (layer "F.Cu") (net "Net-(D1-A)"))
 (segment (start 141.269997 112.295) (end 143.3025 112.295) (width 0.2) (layer "F.Cu") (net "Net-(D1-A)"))
 (segment (start 149.300002 115.769996) (end 144.990006 111.46) (width 0.2) (layer "F.Cu") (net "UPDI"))
 (segment (start 144.990006 111.46) (end 137.23 111.46) (width 0.2) (layer "F.Cu") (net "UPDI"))
 (segment (start 137.23 110.19) (end 140.815 110.19) (width 0.2) (layer "F.Cu") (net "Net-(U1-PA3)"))
 (segment (start 140.815 110.19) (end 141.27 110.645) (width 0.2) (layer "F.Cu") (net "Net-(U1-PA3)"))
 (segment (start 133.555 110.490001) (end 133.254999 110.19) (width 0.2) (layer "F.Cu") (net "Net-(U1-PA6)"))
 (segment (start 132.81 115.82) (end 133.555 115.075) (width 0.2) (layer "F.Cu") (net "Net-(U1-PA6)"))
 (segment (start 133.254999 110.19) (end 132.28 110.19) (width 0.2) (layer "F.Cu") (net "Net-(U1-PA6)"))
 (segment (start 133.555 115.075) (end 133.555 110.490001) (width 0.2) (layer "F.Cu") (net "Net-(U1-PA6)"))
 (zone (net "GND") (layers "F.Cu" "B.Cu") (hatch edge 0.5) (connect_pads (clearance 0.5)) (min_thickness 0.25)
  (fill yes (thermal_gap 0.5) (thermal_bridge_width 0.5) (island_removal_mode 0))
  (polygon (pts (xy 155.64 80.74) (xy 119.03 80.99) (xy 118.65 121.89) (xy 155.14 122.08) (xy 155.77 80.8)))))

